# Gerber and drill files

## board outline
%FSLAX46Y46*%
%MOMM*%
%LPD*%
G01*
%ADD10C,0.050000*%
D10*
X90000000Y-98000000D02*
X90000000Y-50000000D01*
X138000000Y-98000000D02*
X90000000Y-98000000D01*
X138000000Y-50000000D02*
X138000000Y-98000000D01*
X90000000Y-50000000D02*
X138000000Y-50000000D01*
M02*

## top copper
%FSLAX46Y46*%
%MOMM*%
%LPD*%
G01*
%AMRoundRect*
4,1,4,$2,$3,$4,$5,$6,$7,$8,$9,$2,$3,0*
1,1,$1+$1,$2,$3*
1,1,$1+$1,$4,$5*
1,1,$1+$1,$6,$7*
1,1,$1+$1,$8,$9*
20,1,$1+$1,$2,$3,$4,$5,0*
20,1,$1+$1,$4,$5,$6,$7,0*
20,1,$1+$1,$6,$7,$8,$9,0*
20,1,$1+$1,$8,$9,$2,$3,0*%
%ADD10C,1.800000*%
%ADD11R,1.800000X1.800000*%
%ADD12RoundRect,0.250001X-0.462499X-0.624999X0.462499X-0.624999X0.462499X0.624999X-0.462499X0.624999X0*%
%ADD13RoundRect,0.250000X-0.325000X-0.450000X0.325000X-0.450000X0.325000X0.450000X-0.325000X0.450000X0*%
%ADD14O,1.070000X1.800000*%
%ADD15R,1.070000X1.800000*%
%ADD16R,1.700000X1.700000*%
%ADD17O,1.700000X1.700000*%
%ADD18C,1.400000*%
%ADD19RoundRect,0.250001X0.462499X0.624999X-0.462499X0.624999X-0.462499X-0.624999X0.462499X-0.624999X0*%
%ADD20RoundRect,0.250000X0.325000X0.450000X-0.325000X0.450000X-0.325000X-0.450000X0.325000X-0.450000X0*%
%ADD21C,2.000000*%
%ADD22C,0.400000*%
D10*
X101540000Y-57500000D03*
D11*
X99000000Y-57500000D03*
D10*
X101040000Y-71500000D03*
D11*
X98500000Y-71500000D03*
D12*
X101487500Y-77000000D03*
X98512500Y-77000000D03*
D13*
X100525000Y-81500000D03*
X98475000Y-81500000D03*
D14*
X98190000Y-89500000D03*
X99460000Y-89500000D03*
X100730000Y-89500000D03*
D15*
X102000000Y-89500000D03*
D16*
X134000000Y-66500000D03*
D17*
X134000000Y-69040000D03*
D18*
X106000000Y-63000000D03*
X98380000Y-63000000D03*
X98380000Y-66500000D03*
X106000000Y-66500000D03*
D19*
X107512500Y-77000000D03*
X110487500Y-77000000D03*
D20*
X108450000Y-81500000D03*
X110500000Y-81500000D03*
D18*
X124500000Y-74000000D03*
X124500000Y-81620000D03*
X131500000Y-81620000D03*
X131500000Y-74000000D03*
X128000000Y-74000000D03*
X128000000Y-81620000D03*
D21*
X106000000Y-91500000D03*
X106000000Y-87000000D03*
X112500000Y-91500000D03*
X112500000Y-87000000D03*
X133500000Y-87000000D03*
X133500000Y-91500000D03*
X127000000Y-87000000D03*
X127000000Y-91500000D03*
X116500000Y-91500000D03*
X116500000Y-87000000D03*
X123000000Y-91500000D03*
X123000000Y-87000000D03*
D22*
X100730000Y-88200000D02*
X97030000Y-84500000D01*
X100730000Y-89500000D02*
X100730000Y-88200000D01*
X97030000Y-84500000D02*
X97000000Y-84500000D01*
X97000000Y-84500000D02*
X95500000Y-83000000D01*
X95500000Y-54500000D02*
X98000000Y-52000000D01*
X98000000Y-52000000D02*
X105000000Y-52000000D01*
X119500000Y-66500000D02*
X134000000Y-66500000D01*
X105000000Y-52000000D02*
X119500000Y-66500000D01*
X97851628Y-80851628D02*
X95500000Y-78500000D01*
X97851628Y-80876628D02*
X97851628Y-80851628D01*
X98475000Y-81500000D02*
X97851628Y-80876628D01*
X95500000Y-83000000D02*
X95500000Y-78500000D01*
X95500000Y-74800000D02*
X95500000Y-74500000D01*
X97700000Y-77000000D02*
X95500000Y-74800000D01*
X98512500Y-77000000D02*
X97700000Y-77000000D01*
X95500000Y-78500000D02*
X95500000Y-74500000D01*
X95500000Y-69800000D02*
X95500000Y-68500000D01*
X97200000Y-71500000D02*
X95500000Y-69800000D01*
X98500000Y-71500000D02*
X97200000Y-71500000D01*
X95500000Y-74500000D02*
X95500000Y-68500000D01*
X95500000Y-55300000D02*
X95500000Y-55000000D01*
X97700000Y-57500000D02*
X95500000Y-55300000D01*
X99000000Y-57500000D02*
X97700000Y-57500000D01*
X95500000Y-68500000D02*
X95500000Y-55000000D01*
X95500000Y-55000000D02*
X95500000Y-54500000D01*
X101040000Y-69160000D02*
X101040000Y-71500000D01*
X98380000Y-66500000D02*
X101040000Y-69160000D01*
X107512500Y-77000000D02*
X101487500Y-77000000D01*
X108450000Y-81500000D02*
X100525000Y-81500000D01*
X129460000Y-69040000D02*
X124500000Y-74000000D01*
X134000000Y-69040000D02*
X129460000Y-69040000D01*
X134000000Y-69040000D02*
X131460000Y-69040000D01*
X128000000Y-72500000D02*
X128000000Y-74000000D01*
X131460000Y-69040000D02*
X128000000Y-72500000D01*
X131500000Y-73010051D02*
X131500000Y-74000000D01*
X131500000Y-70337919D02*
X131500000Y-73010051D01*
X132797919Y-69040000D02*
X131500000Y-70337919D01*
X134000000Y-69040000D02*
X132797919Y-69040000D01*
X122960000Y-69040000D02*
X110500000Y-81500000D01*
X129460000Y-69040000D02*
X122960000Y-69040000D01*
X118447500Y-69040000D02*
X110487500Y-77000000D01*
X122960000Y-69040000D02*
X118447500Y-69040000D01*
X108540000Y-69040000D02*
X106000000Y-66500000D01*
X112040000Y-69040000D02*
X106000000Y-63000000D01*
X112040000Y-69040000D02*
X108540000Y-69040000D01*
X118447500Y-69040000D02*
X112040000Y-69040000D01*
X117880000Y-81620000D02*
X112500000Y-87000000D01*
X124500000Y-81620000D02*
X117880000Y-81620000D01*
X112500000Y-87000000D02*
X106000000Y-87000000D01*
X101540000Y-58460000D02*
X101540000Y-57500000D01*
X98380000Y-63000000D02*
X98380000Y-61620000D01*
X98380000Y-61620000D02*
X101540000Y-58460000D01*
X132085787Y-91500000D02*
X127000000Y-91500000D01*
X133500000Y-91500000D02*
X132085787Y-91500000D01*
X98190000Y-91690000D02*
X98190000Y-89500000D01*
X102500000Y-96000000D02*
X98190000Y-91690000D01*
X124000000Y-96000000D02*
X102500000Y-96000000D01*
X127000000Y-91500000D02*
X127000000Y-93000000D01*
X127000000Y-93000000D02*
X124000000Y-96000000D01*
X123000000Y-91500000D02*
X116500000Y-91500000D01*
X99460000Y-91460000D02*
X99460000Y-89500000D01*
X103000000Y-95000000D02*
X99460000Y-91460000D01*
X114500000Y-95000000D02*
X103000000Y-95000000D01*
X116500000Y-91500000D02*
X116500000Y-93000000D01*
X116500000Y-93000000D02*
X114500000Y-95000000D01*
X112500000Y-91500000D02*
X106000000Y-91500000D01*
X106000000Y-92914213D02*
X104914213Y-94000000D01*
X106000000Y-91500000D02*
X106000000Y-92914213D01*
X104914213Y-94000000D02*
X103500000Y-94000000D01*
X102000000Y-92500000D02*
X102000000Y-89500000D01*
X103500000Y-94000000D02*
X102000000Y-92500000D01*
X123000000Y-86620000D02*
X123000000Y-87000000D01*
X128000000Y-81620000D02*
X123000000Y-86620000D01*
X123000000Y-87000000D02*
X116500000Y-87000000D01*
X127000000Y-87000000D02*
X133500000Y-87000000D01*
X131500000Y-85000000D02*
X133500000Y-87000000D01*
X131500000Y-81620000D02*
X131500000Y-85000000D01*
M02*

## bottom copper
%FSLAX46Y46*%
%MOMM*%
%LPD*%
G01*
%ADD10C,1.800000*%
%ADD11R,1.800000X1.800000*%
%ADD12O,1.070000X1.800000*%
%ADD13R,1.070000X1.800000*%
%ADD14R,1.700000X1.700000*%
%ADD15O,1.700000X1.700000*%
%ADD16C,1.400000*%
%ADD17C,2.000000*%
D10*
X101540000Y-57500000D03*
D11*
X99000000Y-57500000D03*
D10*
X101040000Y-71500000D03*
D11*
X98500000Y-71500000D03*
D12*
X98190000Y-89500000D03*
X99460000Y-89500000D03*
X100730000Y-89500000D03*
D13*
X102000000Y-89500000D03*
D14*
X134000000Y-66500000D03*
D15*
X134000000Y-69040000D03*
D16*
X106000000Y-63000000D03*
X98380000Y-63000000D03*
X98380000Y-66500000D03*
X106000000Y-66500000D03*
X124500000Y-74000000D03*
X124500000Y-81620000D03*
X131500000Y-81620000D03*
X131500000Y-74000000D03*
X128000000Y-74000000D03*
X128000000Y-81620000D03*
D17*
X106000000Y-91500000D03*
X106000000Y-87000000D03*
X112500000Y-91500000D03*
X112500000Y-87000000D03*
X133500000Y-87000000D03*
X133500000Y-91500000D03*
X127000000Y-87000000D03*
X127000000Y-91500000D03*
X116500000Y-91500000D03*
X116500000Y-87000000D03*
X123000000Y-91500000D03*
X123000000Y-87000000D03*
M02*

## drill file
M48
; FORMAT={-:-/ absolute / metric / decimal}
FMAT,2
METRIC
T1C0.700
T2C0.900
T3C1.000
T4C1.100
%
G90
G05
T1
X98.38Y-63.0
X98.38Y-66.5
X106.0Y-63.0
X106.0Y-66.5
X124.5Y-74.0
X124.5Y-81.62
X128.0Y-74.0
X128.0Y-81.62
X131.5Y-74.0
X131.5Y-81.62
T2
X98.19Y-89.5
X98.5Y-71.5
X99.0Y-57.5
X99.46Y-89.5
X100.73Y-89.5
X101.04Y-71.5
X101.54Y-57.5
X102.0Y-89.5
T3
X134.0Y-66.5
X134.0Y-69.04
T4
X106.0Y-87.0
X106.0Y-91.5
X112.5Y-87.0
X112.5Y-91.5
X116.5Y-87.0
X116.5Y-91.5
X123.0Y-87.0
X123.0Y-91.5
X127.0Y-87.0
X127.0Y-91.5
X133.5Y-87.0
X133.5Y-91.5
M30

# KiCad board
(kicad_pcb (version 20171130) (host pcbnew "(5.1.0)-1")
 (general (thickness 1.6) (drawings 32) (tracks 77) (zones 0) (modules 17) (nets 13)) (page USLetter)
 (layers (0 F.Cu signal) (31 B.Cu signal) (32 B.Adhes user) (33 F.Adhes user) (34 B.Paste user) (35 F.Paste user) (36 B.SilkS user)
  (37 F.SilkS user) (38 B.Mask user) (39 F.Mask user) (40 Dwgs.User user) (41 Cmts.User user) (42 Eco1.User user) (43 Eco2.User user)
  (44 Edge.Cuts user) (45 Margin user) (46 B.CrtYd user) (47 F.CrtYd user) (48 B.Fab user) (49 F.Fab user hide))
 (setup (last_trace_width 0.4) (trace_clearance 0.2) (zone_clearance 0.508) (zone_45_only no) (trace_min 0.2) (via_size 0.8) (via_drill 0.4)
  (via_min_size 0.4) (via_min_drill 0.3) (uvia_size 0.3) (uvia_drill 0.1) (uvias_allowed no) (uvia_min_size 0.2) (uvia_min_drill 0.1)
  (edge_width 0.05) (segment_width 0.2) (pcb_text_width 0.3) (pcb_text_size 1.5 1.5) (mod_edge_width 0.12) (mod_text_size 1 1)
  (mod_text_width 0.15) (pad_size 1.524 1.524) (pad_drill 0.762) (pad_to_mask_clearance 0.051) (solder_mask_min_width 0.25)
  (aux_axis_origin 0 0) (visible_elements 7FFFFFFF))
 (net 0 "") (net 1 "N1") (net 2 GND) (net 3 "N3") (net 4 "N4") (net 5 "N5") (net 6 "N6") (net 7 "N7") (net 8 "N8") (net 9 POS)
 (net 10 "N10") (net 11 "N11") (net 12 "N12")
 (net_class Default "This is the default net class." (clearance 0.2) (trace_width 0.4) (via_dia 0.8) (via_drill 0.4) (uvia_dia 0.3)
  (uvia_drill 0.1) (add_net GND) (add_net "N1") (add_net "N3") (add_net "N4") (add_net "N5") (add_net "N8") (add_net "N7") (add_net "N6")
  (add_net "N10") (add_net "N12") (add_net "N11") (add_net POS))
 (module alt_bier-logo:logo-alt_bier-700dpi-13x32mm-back (layer F.Cu) (at 114 68.5)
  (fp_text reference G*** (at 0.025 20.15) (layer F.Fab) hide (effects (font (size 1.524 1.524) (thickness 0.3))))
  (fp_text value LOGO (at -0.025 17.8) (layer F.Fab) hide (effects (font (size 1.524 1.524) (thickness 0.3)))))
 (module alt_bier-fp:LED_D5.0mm (layer F.Cu) (at 99 57.5)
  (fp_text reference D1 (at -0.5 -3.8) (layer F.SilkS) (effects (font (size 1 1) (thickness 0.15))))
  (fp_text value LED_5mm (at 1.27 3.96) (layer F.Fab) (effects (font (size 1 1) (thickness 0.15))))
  (pad 2 thru_hole circle (at 2.54 0) (size 1.8 1.8) (drill 0.9) (layers *.Cu *.Mask) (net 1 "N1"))
  (pad 1 thru_hole rect (at 0 0) (size 1.8 1.8) (drill 0.9) (layers *.Cu *.Mask) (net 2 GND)))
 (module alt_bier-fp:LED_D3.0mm (layer F.Cu) (at 98.5 71.5)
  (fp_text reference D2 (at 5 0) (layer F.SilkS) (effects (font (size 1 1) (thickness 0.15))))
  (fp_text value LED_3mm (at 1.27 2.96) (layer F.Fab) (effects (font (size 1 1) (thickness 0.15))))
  (pad 2 thru_hole circle (at 2.54 0) (size 1.8 1.8) (drill 0.9) (layers *.Cu *.Mask) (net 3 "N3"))
  (pad 1 thru_hole rect (at 0 0) (size 1.8 1.8) (drill 0.9) (layers *.Cu *.Mask) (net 2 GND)))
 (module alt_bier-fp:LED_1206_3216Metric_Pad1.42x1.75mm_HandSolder (layer F.Cu) (at 100 77)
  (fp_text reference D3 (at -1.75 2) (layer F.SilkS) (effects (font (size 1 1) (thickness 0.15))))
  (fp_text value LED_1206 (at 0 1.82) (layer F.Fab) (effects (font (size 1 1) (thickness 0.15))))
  (pad 2 smd roundrect (at 1.4875 0) (size 1.425 1.75) (layers F.Cu F.Paste F.Mask) (roundrect_rratio 0.175439) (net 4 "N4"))
  (pad 1 smd roundrect (at -1.4875 0) (size 1.425 1.75) (layers F.Cu F.Paste F.Mask) (roundrect_rratio 0.175439) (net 2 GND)))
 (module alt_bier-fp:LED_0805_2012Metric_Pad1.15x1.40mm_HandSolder (layer F.Cu) (at 99.5 81.5)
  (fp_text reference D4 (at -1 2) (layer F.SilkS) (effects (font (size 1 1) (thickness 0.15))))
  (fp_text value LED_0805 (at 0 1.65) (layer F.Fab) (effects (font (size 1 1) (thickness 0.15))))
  (pad 2 smd roundrect (at 1.025 0) (size 1.15 1.4) (layers F.Cu F.Paste F.Mask) (roundrect_rratio 0.217391) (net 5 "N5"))
  (pad 1 smd roundrect (at -1.025 0) (size 1.15 1.4) (layers F.Cu F.Paste F.Mask) (roundrect_rratio 0.217391) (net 2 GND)))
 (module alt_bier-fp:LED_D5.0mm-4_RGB (layer F.Cu) (at 102 89.5 180)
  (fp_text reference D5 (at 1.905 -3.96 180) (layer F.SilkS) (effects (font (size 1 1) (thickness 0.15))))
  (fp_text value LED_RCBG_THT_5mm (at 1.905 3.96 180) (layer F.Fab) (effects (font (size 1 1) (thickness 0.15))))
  (pad 4 thru_hole oval (at 3.81 0 180) (size 1.07 1.8) (drill 0.9) (layers *.Cu *.Mask) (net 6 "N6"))
  (pad 3 thru_hole oval (at 2.54 0 180) (size 1.07 1.8) (drill 0.9) (layers *.Cu *.Mask) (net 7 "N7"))
  (pad 2 thru_hole oval (at 1.27 0 180) (size 1.07 1.8) (drill 0.9) (layers *.Cu *.Mask) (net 2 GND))
  (pad 1 thru_hole rect (at 0 0 180) (size 1.07 1.8) (drill 0.9) (layers *.Cu *.Mask) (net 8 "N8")))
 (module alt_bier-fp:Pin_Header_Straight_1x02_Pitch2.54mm (layer F.Cu) (at 134 66.5)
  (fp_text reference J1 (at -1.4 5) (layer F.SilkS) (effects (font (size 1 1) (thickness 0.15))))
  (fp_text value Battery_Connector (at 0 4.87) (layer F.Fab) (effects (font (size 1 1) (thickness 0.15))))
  (pad 1 thru_hole rect (at 0 0) (size 1.7 1.7) (drill 1) (layers *.Cu *.Mask) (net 2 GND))
  (pad 2 thru_hole oval (at 0 2.54) (size 1.7 1.7) (drill 1) (layers *.Cu *.Mask) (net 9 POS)))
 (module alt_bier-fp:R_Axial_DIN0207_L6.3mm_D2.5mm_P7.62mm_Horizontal (layer F.Cu) (at 106 63 180)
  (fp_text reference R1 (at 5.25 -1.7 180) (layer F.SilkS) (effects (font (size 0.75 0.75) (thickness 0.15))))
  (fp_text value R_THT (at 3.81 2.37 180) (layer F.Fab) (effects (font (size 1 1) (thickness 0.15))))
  (pad 1 thru_hole circle (at 0 0 180) (size 1.4 1.4) (drill 0.7) (layers *.Cu *.Mask) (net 9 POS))
  (pad 2 thru_hole circle (at 7.62 0 180) (size 1.4 1.4) (drill 0.7) (layers *.Cu *.Mask) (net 1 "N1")))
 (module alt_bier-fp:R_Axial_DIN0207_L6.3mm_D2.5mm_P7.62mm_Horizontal (layer F.Cu) (at 106 66.5 180)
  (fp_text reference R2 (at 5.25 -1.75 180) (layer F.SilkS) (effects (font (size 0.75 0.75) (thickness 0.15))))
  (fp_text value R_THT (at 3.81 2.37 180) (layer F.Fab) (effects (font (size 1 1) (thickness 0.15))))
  (pad 2 thru_hole circle (at 7.62 0 180) (size 1.4 1.4) (drill 0.7) (layers *.Cu *.Mask) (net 3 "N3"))
  (pad 1 thru_hole circle (at 0 0 180) (size 1.4 1.4) (drill 0.7) (layers *.Cu *.Mask) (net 9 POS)))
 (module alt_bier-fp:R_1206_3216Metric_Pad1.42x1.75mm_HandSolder (layer F.Cu) (at 109 77 180)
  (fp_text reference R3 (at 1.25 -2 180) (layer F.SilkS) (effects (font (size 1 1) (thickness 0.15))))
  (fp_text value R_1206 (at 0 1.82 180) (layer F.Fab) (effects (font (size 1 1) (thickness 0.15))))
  (pad 2 smd roundrect (at 1.4875 0 180) (size 1.425 1.75) (layers F.Cu F.Paste F.Mask) (roundrect_rratio 0.175439) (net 4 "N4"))
  (pad 1 smd roundrect (at -1.4875 0 180) (size 1.425 1.75) (layers F.Cu F.Paste F.Mask) (roundrect_rratio 0.175439) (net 9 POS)))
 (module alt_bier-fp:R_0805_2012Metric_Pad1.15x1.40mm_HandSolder (layer F.Cu) (at 109.475 81.5 180)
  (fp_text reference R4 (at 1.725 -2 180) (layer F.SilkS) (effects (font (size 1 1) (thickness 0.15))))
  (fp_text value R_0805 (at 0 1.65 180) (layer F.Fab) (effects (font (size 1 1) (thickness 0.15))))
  (pad 2 smd roundrect (at 1.025 0 180) (size 1.15 1.4) (layers F.Cu F.Paste F.Mask) (roundrect_rratio 0.217391) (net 5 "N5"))
  (pad 1 smd roundrect (at -1.025 0 180) (size 1.15 1.4) (layers F.Cu F.Paste F.Mask) (roundrect_rratio 0.217391) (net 9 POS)))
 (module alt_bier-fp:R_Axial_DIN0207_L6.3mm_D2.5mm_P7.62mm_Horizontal (layer F.Cu) (at 124.5 74 270)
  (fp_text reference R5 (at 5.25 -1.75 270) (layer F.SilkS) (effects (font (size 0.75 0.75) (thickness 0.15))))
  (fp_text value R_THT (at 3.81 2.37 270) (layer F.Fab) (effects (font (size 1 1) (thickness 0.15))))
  (pad 1 thru_hole circle (at 0 0 270) (size 1.4 1.4) (drill 0.7) (layers *.Cu *.Mask) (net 9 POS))
  (pad 2 thru_hole circle (at 7.62 0 270) (size 1.4 1.4) (drill 0.7) (layers *.Cu *.Mask) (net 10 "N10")))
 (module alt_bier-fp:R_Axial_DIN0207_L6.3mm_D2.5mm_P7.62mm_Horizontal (layer F.Cu) (at 131.5 74 270)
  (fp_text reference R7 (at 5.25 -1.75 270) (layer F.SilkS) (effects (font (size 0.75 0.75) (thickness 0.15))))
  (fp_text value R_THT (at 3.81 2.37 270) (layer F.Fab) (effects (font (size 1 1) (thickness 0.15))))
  (pad 2 thru_hole circle (at 7.62 0 270) (size 1.4 1.4) (drill 0.7) (layers *.Cu *.Mask) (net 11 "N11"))
  (pad 1 thru_hole circle (at 0 0 270) (size 1.4 1.4) (drill 0.7) (layers *.Cu *.Mask) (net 9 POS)))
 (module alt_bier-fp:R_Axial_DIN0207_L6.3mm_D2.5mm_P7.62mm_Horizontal (layer F.Cu) (at 128 74 270)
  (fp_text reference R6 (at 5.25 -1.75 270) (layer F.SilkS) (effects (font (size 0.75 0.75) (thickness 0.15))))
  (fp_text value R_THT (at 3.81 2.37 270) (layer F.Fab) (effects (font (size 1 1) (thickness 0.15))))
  (pad 1 thru_hole circle (at 0 0 270) (size 1.4 1.4) (drill 0.7) (layers *.Cu *.Mask) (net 9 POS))
  (pad 2 thru_hole circle (at 7.62 0 270) (size 1.4 1.4) (drill 0.7) (layers *.Cu *.Mask) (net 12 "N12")))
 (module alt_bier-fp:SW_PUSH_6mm (layer F.Cu) (at 112.5 91.5 180)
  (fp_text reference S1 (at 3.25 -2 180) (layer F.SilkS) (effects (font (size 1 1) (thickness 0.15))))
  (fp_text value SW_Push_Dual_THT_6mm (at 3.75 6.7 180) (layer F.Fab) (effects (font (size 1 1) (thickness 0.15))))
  (pad 1 thru_hole circle (at 6.5 0 270) (size 2 2) (drill 1.1) (layers *.Cu *.Mask) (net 8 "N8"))
  (pad 2 thru_hole circle (at 6.5 4.5 270) (size 2 2) (drill 1.1) (layers *.Cu *.Mask) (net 10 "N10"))
  (pad 1 thru_hole circle (at 0 0 270) (size 2 2) (drill 1.1) (layers *.Cu *.Mask) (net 8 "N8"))
  (pad 2 thru_hole circle (at 0 4.5 270) (size 2 2) (drill 1.1) (layers *.Cu *.Mask) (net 10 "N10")))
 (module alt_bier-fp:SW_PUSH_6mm (layer F.Cu) (at 133.5 91.5 180)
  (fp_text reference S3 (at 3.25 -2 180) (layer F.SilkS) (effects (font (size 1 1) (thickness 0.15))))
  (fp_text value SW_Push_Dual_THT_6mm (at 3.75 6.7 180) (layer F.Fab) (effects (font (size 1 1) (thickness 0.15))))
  (pad 2 thru_hole circle (at 0 4.5 270) (size 2 2) (drill 1.1) (layers *.Cu *.Mask) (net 11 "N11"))
  (pad 1 thru_hole circle (at 0 0 270) (size 2 2) (drill 1.1) (layers *.Cu *.Mask) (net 6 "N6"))
  (pad 2 thru_hole circle (at 6.5 4.5 270) (size 2 2) (drill 1.1) (layers *.Cu *.Mask) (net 11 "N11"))
  (pad 1 thru_hole circle (at 6.5 0 270) (size 2 2) (drill 1.1) (layers *.Cu *.Mask) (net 6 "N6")))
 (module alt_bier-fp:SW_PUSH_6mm (layer F.Cu) (at 123 91.5 180)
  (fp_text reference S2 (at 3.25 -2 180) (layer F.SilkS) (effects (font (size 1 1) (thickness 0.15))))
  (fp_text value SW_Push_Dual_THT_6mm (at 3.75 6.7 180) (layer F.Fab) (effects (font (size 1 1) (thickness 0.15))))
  (pad 1 thru_hole circle (at 6.5 0 270) (size 2 2) (drill 1.1) (layers *.Cu *.Mask) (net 7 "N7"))
  (pad 2 thru_hole circle (at 6.5 4.5 270) (size 2 2) (drill 1.1) (layers *.Cu *.Mask) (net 12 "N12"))
  (pad 1 thru_hole circle (at 0 0 270) (size 2 2) (drill 1.1) (layers *.Cu *.Mask) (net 7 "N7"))
  (pad 2 thru_hole circle (at 0 4.5 270) (size 2 2) (drill 1.1) (layers *.Cu *.Mask) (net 12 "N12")))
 (gr_line (start 90 98) (end 90 50) (layer Edge.Cuts) (width 0.05))
 (gr_line (start 138 98) (end 90 98) (layer Edge.Cuts) (width 0.05))
 (gr_line (start 138 50) (end 138 98) (layer Edge.Cuts) (width 0.05))
 (gr_line (start 90 50) (end 138 50) (layer Edge.Cuts) (width 0.05))
 (segment (start 100.73 88.2) (end 97.03 84.5) (width 0.4) (layer F.Cu) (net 2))
 (segment (start 100.73 89.5) (end 100.73 88.2) (width 0.4) (layer F.Cu) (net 2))
 (segment (start 97.03 84.5) (end 97 84.5) (width 0.4) (layer F.Cu) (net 2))
 (segment (start 97 84.5) (end 95.5 83) (width 0.4) (layer F.Cu) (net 2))
 (segment (start 95.5 54.5) (end 98 52) (width 0.4) (layer F.Cu) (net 2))
 (segment (start 98 52) (end 105 52) (width 0.4) (layer F.Cu) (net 2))
 (segment (start 119.5 66.5) (end 134 66.5) (width 0.4) (layer F.Cu) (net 2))
 (segment (start 105 52) (end 119.5 66.5) (width 0.4) (layer F.Cu) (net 2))
 (segment (start 97.851628 80.851628) (end 95.5 78.5) (width 0.4) (layer F.Cu) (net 2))
 (segment (start 97.851628 80.876628) (end 97.851628 80.851628) (width 0.4) (layer F.Cu) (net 2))
 (segment (start 98.475 81.5) (end 97.851628 80.876628) (width 0.4) (layer F.Cu) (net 2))
 (segment (start 95.5 83) (end 95.5 78.5) (width 0.4) (layer F.Cu) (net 2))
 (segment (start 95.5 74.8) (end 95.5 74.5) (width 0.4) (layer F.Cu) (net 2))
 (segment (start 97.7 77) (end 95.5 74.8) (width 0.4) (layer F.Cu) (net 2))
 (segment (start 98.5125 77) (end 97.7 77) (width 0.4) (layer F.Cu) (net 2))
 (segment (start 95.5 78.5) (end 95.5 74.5) (width 0.4) (layer F.Cu) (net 2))
 (segment (start 95.5 69.8) (end 95.5 68.5) (width 0.4) (layer F.Cu) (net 2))
 (segment (start 97.2 71.5) (end 95.5 69.8) (width 0.4) (layer F.Cu) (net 2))
 (segment (start 98.5 71.5) (end 97.2 71.5) (width 0.4) (layer F.Cu) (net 2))
 (segment (start 95.5 74.5) (end 95.5 68.5) (width 0.4) (layer F.Cu) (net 2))
 (segment (start 95.5 55.3) (end 95.5 55) (width 0.4) (layer F.Cu) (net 2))
 (segment (start 97.7 57.5) (end 95.5 55.3) (width 0.4) (layer F.Cu) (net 2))
 (segment (start 99 57.5) (end 97.7 57.5) (width 0.4) (layer F.Cu) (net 2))
 (segment (start 95.5 68.5) (end 95.5 55) (width 0.4) (layer F.Cu) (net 2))
 (segment (start 95.5 55) (end 95.5 54.5) (width 0.4) (layer F.Cu) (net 2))
 (segment (start 101.04 69.16) (end 101.04 71.5) (width 0.4) (layer F.Cu) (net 3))
 (segment (start 98.38 66.5) (end 101.04 69.16) (width 0.4) (layer F.Cu) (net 3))
 (segment (start 107.5125 77) (end 101.4875 77) (width 0.4) (layer F.Cu) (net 4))
 (segment (start 108.45 81.5) (end 100.525 81.5) (width 0.4) (layer F.Cu) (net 5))
 (segment (start 129.46 69.04) (end 124.5 74) (width 0.4) (layer F.Cu) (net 9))
 (segment (start 134 69.04) (end 129.46 69.04) (width 0.4) (layer F.Cu) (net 9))
 (segment (start 134 69.04) (end 131.46 69.04) (width 0.4) (layer F.Cu) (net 9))
 (segment (start 128 72.5) (end 128 74) (width 0.4) (layer F.Cu) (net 9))
 (segment (start 131.46 69.04) (end 128 72.5) (width 0.4) (layer F.Cu) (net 9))
 (segment (start 131.5 73.010051) (end 131.5 74) (width 0.4) (layer F.Cu) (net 9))
 (segment (start 131.5 70.337919) (end 131.5 73.010051) (width 0.4) (layer F.Cu) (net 9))
 (segment (start 132.797919 69.04) (end 131.5 70.337919) (width 0.4) (layer F.Cu) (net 9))
 (segment (start 134 69.04) (end 132.797919 69.04) (width 0.4) (layer F.Cu) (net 9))
 (segment (start 122.96 69.04) (end 110.5 81.5) (width 0.4) (layer F.Cu) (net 9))
 (segment (start 129.46 69.04) (end 122.96 69.04) (width 0.4) (layer F.Cu) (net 9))
 (segment (start 118.4475 69.04) (end 110.4875 77) (width 0.4) (layer F.Cu) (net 9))
 (segment (start 122.96 69.04) (end 118.4475 69.04) (width 0.4) (layer F.Cu) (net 9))
 (segment (start 108.54 69.04) (end 106 66.5) (width 0.4) (layer F.Cu) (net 9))
 (segment (start 112.04 69.04) (end 106 63) (width 0.4) (layer F.Cu) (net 9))
 (segment (start 112.04 69.04) (end 108.54 69.04) (width 0.4) (layer F.Cu) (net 9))
 (segment (start 118.4475 69.04) (end 112.04 69.04) (width 0.4) (layer F.Cu) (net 9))
 (segment (start 117.88 81.62) (end 112.5 87) (width 0.4) (layer F.Cu) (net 10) (status 20))
 (segment (start 124.5 81.62) (end 117.88 81.62) (width 0.4) (layer F.Cu) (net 10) (status 10))
 (segment (start 112.5 87) (end 106 87) (width 0.4) (layer F.Cu) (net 10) (status 30))
 (segment (start 101.54 58.46) (end 101.54 57.5) (width 0.4) (layer F.Cu) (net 1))
 (segment (start 98.38 63) (end 98.38 61.62) (width 0.4) (layer F.Cu) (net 1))
 (segment (start 98.38 61.62) (end 101.54 58.46) (width 0.4) (layer F.Cu) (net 1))
 (segment (start 132.085787 91.5) (end 127 91.5) (width 0.4) (layer F.Cu) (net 6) (status 20))
 (segment (start 133.5 91.5) (end 132.085787 91.5) (width 0.4) (layer F.Cu) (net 6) (status 10))
 (segment (start 98.19 91.69) (end 98.19 89.5) (width 0.4) (layer F.Cu) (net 6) (status 20))
 (segment (start 102.5 96) (end 98.19 91.69) (width 0.4) (layer F.Cu) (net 6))
 (segment (start 124 96) (end 102.5 96) (width 0.4) (layer F.Cu) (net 6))
 (segment (start 127 91.5) (end 127 93) (width 0.4) (layer F.Cu) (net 6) (status 10))
 (segment (start 127 93) (end 124 96) (width 0.4) (layer F.Cu) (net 6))
 (segment (start 123 91.5) (end 116.5 91.5) (width 0.4) (layer F.Cu) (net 7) (status 30))
 (segment (start 99.46 91.46) (end 99.46 89.5) (width 0.4) (layer F.Cu) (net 7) (status 20))
 (segment (start 103 95) (end 99.46 91.46) (width 0.4) (layer F.Cu) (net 7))
 (segment (start 114.5 95) (end 103 95) (width 0.4) (layer F.Cu) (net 7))
 (segment (start 116.5 91.5) (end 116.5 93) (width 0.4) (layer F.Cu) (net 7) (status 10))
 (segment (start 116.5 93) (end 114.5 95) (width 0.4) (layer F.Cu) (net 7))
 (segment (start 112.5 91.5) (end 106 91.5) (width 0.4) (layer F.Cu) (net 8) (status 30))
 (segment (start 106 92.914213) (end 104.914213 94) (width 0.4) (layer F.Cu) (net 8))
 (segment (start 106 91.5) (end 106 92.914213) (width 0.4) (layer F.Cu) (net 8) (status 10))
 (segment (start 104.914213 94) (end 103.5 94) (width 0.4) (layer F.Cu) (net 8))
 (segment (start 102 92.5) (end 102 89.5) (width 0.4) (layer F.Cu) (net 8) (status 20))
 (segment (start 103.5 94) (end 102 92.5) (width 0.4) (layer F.Cu) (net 8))
 (segment (start 123 86.62) (end 123 87) (width 0.4) (layer F.Cu) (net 12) (status 30))
 (segment (start 128 81.62) (end 123 86.62) (width 0.4) (layer F.Cu) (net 12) (status 30))
 (segment (start 123 87) (end 116.5 87) (width 0.4) (layer F.Cu) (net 12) (status 30))
 (segment (start 127 87) (end 133.5 87) (width 0.4) (layer F.Cu) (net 11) (status 30))
 (segment (start 131.5 85) (end 133.5 87) (width 0.4) (layer F.Cu) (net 11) (status 20))
 (segment (start 131.5 81.62) (end 131.5 85) (width 0.4) (layer F.Cu) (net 11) (status 10)))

